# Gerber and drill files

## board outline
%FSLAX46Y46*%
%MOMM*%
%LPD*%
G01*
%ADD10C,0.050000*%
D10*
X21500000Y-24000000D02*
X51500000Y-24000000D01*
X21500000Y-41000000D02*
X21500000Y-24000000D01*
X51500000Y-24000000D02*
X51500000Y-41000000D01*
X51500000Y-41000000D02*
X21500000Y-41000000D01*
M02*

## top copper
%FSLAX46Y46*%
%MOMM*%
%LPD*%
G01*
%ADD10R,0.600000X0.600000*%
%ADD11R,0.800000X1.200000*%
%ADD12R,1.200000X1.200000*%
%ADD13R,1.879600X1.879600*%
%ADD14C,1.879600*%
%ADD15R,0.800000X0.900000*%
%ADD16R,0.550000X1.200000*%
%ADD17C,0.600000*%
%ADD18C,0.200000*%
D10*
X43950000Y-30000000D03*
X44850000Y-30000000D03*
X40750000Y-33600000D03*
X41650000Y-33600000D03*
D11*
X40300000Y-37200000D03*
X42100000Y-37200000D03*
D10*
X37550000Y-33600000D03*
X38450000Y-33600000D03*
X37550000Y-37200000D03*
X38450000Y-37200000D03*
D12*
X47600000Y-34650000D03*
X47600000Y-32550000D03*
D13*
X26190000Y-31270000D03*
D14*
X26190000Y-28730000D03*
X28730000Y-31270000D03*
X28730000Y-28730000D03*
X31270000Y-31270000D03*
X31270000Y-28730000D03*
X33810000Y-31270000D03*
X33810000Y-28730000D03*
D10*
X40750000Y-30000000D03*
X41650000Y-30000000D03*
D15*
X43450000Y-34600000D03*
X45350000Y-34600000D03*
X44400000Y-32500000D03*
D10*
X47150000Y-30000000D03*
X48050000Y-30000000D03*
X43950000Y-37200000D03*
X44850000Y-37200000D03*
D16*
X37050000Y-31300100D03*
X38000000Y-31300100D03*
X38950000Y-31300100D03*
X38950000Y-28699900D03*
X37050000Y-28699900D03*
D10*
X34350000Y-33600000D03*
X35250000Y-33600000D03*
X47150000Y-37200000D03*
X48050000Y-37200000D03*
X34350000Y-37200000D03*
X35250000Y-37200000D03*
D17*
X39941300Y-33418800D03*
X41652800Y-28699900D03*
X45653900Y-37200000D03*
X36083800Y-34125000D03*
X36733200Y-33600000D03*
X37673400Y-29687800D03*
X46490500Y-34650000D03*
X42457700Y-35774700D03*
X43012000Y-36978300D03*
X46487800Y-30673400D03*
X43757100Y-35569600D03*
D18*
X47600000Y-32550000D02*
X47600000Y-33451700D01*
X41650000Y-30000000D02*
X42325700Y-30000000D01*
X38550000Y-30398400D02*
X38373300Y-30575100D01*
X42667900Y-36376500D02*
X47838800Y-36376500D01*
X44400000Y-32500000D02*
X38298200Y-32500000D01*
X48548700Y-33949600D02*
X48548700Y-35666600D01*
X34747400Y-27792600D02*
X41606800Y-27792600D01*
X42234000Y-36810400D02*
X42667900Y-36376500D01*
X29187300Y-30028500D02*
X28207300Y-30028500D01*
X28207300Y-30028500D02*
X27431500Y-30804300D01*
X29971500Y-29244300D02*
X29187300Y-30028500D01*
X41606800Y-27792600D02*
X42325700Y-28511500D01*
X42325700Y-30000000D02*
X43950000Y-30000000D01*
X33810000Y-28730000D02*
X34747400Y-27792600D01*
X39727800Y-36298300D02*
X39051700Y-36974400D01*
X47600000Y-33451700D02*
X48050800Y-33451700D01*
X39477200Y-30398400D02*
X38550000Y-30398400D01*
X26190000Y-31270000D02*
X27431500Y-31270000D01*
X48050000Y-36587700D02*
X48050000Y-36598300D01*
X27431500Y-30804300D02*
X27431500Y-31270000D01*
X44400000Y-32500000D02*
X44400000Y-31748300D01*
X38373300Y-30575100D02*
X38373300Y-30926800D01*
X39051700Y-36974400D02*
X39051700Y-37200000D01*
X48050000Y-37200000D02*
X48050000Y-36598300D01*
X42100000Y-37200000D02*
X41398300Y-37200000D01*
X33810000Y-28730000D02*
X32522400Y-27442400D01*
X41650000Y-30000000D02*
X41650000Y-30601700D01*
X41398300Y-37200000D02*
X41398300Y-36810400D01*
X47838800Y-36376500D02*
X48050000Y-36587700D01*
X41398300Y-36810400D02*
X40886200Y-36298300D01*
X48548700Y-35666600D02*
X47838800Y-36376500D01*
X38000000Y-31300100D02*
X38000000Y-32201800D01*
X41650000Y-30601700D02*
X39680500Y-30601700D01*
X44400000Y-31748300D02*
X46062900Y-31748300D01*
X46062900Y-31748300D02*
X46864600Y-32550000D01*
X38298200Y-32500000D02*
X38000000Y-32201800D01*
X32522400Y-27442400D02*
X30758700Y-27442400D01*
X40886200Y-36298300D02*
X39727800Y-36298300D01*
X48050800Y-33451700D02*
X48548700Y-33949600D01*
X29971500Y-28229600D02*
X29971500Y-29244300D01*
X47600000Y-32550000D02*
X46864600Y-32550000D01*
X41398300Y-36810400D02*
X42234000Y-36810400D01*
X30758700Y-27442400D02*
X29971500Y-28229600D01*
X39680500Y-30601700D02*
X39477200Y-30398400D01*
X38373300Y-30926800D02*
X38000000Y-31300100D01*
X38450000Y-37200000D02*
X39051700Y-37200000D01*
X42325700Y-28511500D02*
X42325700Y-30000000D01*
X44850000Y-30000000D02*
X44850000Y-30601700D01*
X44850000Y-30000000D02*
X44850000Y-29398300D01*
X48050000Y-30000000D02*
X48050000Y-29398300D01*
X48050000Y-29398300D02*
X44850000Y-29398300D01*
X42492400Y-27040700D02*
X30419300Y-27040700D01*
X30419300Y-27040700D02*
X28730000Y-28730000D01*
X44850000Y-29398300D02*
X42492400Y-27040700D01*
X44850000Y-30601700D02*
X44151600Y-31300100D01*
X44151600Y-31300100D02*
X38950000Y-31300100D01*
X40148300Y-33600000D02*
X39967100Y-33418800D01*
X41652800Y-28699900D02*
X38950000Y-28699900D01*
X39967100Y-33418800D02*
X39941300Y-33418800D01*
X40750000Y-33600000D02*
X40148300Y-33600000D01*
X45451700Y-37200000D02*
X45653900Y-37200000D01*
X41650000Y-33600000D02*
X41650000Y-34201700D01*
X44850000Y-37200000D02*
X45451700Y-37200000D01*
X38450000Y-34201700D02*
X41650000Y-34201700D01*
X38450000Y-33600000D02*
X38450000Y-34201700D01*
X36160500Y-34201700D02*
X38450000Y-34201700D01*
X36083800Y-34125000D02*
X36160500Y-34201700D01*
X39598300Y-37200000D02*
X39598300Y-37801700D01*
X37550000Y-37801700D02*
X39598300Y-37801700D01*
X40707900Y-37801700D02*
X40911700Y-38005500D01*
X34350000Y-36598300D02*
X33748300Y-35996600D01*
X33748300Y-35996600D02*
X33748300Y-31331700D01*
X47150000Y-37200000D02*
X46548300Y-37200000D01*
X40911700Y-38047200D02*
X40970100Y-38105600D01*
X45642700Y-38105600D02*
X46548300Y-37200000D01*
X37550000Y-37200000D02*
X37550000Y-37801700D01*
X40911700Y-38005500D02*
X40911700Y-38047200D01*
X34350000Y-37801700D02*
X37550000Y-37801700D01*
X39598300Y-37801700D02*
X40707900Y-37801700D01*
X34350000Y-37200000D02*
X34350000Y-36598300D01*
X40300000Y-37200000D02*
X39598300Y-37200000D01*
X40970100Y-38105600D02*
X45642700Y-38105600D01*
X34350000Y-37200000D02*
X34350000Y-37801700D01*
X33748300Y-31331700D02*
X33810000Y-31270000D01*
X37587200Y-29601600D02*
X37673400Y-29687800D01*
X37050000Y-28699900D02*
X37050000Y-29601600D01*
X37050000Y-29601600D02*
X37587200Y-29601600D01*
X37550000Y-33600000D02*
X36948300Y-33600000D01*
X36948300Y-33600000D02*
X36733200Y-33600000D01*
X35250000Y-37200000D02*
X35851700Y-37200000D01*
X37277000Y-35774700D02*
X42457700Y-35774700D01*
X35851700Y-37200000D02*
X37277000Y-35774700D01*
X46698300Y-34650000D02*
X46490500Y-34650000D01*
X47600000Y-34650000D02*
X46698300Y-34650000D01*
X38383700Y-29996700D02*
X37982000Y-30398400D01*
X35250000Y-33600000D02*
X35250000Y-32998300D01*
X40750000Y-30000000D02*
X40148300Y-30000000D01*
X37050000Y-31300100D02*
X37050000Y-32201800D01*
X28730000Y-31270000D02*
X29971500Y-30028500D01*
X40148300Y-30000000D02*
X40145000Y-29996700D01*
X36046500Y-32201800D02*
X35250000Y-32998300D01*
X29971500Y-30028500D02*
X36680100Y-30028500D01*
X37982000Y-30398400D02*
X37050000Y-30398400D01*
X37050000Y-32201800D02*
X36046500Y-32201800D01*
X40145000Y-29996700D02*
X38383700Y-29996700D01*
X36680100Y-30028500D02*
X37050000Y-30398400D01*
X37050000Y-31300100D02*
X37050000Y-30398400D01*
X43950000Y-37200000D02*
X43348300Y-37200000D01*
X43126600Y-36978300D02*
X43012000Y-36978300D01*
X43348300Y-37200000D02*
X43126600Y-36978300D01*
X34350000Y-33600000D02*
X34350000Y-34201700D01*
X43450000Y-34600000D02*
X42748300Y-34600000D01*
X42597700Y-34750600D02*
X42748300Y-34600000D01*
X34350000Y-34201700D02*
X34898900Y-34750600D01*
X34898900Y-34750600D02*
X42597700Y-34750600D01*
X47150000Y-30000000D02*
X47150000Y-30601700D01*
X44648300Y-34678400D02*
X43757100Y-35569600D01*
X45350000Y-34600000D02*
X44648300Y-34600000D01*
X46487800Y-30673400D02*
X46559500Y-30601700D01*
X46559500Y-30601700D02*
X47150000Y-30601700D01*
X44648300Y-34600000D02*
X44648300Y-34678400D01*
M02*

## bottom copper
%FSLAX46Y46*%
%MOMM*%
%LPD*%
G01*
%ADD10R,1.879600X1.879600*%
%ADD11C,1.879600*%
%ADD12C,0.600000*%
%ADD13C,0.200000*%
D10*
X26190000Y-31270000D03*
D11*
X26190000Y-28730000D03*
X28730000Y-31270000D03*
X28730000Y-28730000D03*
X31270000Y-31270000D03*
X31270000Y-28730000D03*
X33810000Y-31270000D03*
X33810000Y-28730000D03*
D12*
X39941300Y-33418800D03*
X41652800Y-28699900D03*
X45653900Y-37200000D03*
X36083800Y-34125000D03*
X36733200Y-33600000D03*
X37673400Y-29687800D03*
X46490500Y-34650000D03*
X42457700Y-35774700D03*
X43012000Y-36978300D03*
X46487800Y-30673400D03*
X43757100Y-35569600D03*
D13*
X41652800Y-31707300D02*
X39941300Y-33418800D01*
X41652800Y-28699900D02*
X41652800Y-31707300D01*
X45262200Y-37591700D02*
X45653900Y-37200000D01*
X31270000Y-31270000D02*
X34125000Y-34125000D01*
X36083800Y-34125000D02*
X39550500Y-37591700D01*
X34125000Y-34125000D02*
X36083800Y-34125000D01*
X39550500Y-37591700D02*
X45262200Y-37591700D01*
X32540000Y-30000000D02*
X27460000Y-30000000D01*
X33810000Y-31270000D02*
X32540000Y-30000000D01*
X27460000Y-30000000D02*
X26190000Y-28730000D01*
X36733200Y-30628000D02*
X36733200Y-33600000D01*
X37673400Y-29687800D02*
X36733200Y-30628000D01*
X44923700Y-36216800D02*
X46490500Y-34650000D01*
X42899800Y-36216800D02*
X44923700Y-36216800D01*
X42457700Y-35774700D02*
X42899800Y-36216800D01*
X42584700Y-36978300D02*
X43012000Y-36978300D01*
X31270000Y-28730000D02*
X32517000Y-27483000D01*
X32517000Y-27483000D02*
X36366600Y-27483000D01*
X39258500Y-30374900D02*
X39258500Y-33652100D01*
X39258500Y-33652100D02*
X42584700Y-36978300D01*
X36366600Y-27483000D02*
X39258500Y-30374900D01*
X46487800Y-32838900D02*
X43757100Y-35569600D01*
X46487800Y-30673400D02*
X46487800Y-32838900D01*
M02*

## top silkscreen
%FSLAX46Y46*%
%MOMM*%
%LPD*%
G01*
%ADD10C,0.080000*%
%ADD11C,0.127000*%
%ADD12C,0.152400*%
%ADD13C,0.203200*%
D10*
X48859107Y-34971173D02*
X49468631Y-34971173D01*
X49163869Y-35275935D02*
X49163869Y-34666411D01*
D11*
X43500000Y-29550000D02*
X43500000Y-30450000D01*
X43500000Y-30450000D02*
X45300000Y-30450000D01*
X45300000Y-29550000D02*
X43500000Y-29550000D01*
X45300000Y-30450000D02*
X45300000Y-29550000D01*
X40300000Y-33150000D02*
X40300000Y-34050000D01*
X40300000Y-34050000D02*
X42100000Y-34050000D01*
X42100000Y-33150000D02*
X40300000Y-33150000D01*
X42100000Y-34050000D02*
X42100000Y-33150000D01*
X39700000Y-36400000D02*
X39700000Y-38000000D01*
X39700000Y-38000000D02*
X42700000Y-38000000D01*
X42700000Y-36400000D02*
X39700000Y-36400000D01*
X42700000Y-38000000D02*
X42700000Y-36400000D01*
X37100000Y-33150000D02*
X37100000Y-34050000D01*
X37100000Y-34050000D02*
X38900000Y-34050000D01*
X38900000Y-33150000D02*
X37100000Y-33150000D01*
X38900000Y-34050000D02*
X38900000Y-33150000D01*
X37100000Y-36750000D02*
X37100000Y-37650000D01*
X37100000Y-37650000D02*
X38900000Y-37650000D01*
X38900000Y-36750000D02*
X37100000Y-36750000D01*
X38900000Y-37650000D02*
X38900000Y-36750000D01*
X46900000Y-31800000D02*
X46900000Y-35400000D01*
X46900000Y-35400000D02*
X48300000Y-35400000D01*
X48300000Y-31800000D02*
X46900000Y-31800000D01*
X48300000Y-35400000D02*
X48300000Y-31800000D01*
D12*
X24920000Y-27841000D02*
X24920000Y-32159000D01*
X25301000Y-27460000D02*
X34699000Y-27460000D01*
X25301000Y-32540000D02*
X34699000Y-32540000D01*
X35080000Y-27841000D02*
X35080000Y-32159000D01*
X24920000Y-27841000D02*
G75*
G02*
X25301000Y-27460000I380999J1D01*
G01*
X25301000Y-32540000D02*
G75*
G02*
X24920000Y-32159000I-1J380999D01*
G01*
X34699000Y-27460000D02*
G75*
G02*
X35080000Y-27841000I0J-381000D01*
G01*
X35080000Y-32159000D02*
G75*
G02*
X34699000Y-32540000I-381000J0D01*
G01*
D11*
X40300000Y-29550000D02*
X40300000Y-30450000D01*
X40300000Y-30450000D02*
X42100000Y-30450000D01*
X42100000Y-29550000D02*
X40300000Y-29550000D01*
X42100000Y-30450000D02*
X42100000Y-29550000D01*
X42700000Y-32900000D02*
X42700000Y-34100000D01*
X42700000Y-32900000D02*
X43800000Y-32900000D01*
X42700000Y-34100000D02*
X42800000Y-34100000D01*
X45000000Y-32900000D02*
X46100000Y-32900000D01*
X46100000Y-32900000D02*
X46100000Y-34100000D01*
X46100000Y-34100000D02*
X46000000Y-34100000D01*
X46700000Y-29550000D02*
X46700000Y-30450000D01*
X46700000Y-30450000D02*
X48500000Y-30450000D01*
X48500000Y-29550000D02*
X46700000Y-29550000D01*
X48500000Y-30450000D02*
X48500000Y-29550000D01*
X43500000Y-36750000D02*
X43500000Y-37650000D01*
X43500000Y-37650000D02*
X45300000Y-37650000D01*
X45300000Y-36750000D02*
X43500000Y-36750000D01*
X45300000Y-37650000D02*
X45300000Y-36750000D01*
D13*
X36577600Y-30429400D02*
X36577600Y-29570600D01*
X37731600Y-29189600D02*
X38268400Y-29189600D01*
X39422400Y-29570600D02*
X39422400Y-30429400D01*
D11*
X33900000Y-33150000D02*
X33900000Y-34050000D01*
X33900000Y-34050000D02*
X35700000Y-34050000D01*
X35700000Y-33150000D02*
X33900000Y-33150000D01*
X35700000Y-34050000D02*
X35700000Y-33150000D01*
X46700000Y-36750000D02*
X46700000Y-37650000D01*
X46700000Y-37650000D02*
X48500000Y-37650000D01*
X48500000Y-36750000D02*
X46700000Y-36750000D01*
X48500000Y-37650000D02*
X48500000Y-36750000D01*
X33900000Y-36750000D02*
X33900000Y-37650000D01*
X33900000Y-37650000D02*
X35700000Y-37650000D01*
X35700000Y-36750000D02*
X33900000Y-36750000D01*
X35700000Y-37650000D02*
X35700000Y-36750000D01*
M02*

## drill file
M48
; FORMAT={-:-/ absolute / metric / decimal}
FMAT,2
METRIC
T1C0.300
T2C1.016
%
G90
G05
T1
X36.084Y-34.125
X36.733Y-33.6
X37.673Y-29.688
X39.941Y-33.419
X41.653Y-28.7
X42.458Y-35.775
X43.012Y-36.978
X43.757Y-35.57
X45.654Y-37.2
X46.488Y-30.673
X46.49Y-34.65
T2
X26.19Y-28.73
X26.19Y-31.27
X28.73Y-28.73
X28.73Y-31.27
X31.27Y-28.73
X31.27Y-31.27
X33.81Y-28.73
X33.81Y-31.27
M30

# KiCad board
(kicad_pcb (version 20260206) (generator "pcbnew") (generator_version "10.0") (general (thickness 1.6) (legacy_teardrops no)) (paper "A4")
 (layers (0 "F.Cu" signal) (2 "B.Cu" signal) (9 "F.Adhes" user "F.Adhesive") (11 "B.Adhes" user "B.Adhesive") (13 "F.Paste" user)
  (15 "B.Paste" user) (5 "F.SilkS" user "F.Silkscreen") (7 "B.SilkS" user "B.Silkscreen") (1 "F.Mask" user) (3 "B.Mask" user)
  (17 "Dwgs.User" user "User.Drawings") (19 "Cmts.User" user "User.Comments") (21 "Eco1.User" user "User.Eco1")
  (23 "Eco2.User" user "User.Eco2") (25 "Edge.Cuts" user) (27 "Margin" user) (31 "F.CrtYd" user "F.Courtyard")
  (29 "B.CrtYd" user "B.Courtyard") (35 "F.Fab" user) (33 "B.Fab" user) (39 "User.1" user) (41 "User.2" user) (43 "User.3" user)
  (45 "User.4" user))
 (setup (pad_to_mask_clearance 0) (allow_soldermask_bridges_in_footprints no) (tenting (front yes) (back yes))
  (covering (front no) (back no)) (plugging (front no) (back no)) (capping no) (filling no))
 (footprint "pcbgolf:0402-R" (layer "F.Cu") (at 44.4 30)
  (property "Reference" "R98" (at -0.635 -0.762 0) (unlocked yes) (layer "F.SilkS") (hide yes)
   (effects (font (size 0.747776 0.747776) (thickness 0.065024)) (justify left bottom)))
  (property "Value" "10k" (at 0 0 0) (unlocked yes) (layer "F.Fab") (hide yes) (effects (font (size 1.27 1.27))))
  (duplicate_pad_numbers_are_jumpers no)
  (fp_line (start -0.9 -0.45) (end -0.9 0.45) (stroke (width 0.127) (type solid)) (layer "F.SilkS"))
  (fp_line (start -0.9 0.45) (end 0.9 0.45) (stroke (width 0.127) (type solid)) (layer "F.SilkS"))
  (fp_line (start 0.9 -0.45) (end -0.9 -0.45) (stroke (width 0.127) (type solid)) (layer "F.SilkS"))
  (fp_line (start 0.9 0.45) (end 0.9 -0.45) (stroke (width 0.127) (type solid)) (layer "F.SilkS"))
  (pad "1" smd rect (at -0.45 0) (size 0.6 0.6) (layers "F.Cu" "F.Mask" "F.Paste") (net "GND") (solder_mask_margin 0.0508)
   (solder_paste_margin 0) (thermal_bridge_angle 0))
  (pad "2" smd rect (at 0.45 0) (size 0.6 0.6) (layers "F.Cu" "F.Mask" "F.Paste") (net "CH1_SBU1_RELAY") (solder_mask_margin 0.0508)
   (solder_paste_margin 0) (thermal_bridge_angle 0)))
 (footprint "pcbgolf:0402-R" (layer "F.Cu") (at 41.2 33.6)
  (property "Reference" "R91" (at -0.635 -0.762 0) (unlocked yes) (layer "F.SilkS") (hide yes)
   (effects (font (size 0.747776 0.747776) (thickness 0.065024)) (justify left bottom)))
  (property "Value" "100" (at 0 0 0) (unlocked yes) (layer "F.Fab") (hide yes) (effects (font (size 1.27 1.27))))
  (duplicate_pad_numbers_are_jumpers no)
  (fp_line (start -0.9 -0.45) (end -0.9 0.45) (stroke (width 0.127) (type solid)) (layer "F.SilkS"))
  (fp_line (start -0.9 0.45) (end 0.9 0.45) (stroke (width 0.127) (type solid)) (layer "F.SilkS"))
  (fp_line (start 0.9 -0.45) (end -0.9 -0.45) (stroke (width 0.127) (type solid)) (layer "F.SilkS"))
  (fp_line (start 0.9 0.45) (end 0.9 -0.45) (stroke (width 0.127) (type solid)) (layer "F.SilkS"))
  (pad "1" smd rect (at -0.45 0) (size 0.6 0.6) (layers "F.Cu" "F.Mask" "F.Paste") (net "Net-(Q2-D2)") (solder_mask_margin 0.0508)
   (solder_paste_margin 0) (thermal_bridge_angle 0))
  (pad "2" smd rect (at 0.45 0) (size 0.6 0.6) (layers "F.Cu" "F.Mask" "F.Paste") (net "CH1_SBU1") (solder_mask_margin 0.0508)
   (solder_paste_margin 0) (thermal_bridge_angle 0)))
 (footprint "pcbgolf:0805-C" (layer "F.Cu") (at 41.2 37.2)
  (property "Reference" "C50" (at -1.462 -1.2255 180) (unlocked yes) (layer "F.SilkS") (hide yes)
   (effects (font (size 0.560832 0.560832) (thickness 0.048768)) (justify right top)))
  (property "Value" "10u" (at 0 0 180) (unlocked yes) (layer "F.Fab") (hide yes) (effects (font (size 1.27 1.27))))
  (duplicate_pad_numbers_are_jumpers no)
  (fp_line (start -1.5 -0.8) (end -1.5 0.8) (stroke (width 0.127) (type solid)) (layer "F.SilkS"))
  (fp_line (start -1.5 0.8) (end 1.5 0.8) (stroke (width 0.127) (type solid)) (layer "F.SilkS"))
  (fp_line (start 1.5 -0.8) (end -1.5 -0.8) (stroke (width 0.127) (type solid)) (layer "F.SilkS"))
  (fp_line (start 1.5 0.8) (end 1.5 -0.8) (stroke (width 0.127) (type solid)) (layer "F.SilkS"))
  (pad "1" smd rect (at -0.9 0) (size 0.8 1.2) (layers "F.Cu" "F.Mask" "F.Paste") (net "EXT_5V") (solder_mask_margin 0.0508)
   (solder_paste_margin 0) (thermal_bridge_angle 0))
  (pad "2" smd rect (at 0.9 0) (size 0.8 1.2) (layers "F.Cu" "F.Mask" "F.Paste") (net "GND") (solder_mask_margin 0.0508)
   (solder_paste_margin 0) (thermal_bridge_angle 0)))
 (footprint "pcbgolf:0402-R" (layer "F.Cu") (at 38 33.6)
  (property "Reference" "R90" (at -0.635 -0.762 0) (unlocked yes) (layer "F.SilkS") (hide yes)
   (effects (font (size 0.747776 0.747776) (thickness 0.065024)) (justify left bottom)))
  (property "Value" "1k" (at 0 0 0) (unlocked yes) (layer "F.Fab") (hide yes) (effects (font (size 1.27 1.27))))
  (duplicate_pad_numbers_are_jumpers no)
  (fp_line (start -0.9 -0.45) (end -0.9 0.45) (stroke (width 0.127) (type solid)) (layer "F.SilkS"))
  (fp_line (start -0.9 0.45) (end 0.9 0.45) (stroke (width 0.127) (type solid)) (layer "F.SilkS"))
  (fp_line (start 0.9 -0.45) (end -0.9 -0.45) (stroke (width 0.127) (type solid)) (layer "F.SilkS"))
  (fp_line (start 0.9 0.45) (end 0.9 -0.45) (stroke (width 0.127) (type solid)) (layer "F.SilkS"))
  (pad "1" smd rect (at -0.45 0) (size 0.6 0.6) (layers "F.Cu" "F.Mask" "F.Paste") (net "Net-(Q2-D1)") (solder_mask_margin 0.0508)
   (solder_paste_margin 0) (thermal_bridge_angle 0))
  (pad "2" smd rect (at 0.45 0) (size 0.6 0.6) (layers "F.Cu" "F.Mask" "F.Paste") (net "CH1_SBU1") (solder_mask_margin 0.0508)
   (solder_paste_margin 0) (thermal_bridge_angle 0)))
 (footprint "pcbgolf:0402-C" (layer "F.Cu") (at 38 37.2)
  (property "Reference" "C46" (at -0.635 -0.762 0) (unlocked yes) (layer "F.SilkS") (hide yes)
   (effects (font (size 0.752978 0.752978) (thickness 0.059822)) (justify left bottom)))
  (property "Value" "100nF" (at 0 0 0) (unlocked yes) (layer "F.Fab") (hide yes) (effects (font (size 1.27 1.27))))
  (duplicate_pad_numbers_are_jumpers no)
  (fp_line (start -0.9 -0.45) (end -0.9 0.45) (stroke (width 0.127) (type solid)) (layer "F.SilkS"))
  (fp_line (start -0.9 0.45) (end 0.9 0.45) (stroke (width 0.127) (type solid)) (layer "F.SilkS"))
  (fp_line (start 0.9 -0.45) (end -0.9 -0.45) (stroke (width 0.127) (type solid)) (layer "F.SilkS"))
  (fp_line (start 0.9 0.45) (end 0.9 -0.45) (stroke (width 0.127) (type solid)) (layer "F.SilkS"))
  (pad "1" smd rect (at -0.45 0) (size 0.6 0.6) (layers "F.Cu" "F.Mask" "F.Paste") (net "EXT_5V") (solder_mask_margin 0.0508)
   (solder_paste_margin 0) (thermal_bridge_angle 0))
  (pad "2" smd rect (at 0.45 0) (size 0.6 0.6) (layers "F.Cu" "F.Mask" "F.Paste") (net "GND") (solder_mask_margin 0.0508)
   (solder_paste_margin 0) (thermal_bridge_angle 0)))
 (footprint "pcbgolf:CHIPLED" (layer "F.Cu") (at 47.6 33.6)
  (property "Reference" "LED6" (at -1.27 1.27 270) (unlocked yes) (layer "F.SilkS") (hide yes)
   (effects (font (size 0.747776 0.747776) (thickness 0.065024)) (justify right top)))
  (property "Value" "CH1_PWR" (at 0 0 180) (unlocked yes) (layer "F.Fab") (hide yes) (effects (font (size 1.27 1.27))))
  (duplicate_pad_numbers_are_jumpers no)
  (fp_line (start -0.7 -1.8) (end -0.7 1.8) (stroke (width 0.127) (type solid)) (layer "F.SilkS"))
  (fp_line (start -0.7 1.8) (end 0.7 1.8) (stroke (width 0.127) (type solid)) (layer "F.SilkS"))
  (fp_line (start 0.7 -1.8) (end -0.7 -1.8) (stroke (width 0.127) (type solid)) (layer "F.SilkS"))
  (fp_line (start 0.7 1.8) (end 0.7 -1.8) (stroke (width 0.127) (type solid)) (layer "F.SilkS"))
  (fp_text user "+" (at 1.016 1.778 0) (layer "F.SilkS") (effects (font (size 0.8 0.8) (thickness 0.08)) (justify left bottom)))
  (pad "A" smd rect (at 0 1.05) (size 1.2 1.2) (layers "F.Cu" "F.Mask" "F.Paste") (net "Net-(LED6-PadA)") (solder_mask_margin 0.0508)
   (solder_paste_margin 0) (thermal_bridge_angle 0))
  (pad "C" smd rect (at 0 -1.05) (size 1.2 1.2) (layers "F.Cu" "F.Mask" "F.Paste") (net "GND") (solder_mask_margin 0.0508)
   (solder_paste_margin 0) (thermal_bridge_angle 0)))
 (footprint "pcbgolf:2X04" (layer "F.Cu") (at 30 30)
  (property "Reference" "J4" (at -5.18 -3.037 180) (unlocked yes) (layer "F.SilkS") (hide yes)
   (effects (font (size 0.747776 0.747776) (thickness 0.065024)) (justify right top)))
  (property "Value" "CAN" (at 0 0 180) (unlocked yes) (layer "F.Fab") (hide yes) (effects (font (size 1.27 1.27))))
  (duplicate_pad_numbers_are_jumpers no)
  (fp_line (start -5.08 -2.159) (end -5.08 2.159) (stroke (width 0.1524) (type solid)) (layer "F.SilkS"))
  (fp_line (start -4.699 -2.54) (end 4.699 -2.54) (stroke (width 0.1524) (type solid)) (layer "F.SilkS"))
  (fp_line (start -4.699 2.54) (end 4.699 2.54) (stroke (width 0.1524) (type solid)) (layer "F.SilkS"))
  (fp_line (start 5.08 -2.159) (end 5.08 2.159) (stroke (width 0.1524) (type solid)) (layer "F.SilkS"))
  (fp_arc (start -5.08 -2.159) (mid -4.968408 -2.428408) (end -4.699 -2.54) (stroke (width 0.1524) (type solid)) (layer "F.SilkS"))
  (fp_arc (start -4.699 2.54) (mid -4.968408 2.428408) (end -5.08 2.159) (stroke (width 0.1524) (type solid)) (layer "F.SilkS"))
  (fp_arc (start 4.699 -2.54) (mid 4.968408 -2.428408) (end 5.08 -2.159) (stroke (width 0.1524) (type solid)) (layer "F.SilkS"))
  (fp_arc (start 5.08 2.159) (mid 4.968408 2.428408) (end 4.699 2.54) (stroke (width 0.1524) (type solid)) (layer "F.SilkS"))
  (pad "1" thru_hole rect (at -3.81 1.27 90) (size 1.8796 1.8796) (drill 1.016) (layers "*.Cu" "*.Mask") (remove_unused_layers no)
   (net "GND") (solder_mask_margin 0.0508) (thermal_bridge_angle 0))
  (pad "2" thru_hole circle (at -3.81 -1.27 90) (size 1.8796 1.8796) (drill 1.016) (layers "*.Cu" "*.Mask") (remove_unused_layers no)
   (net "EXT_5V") (solder_mask_margin 0.0508) (thermal_bridge_angle 0))
  (pad "3" thru_hole circle (at -1.27 1.27 90) (size 1.8796 1.8796) (drill 1.016) (layers "*.Cu" "*.Mask") (remove_unused_layers no)
   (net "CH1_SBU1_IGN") (solder_mask_margin 0.0508) (thermal_bridge_angle 0))
  (pad "4" thru_hole circle (at -1.27 -1.27 90) (size 1.8796 1.8796) (drill 1.016) (layers "*.Cu" "*.Mask") (remove_unused_layers no)
   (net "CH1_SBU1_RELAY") (solder_mask_margin 0.0508) (thermal_bridge_angle 0))
  (pad "5" thru_hole circle (at 1.27 1.27 90) (size 1.8796 1.8796) (drill 1.016) (layers "*.Cu" "*.Mask") (remove_unused_layers no)
   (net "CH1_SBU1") (solder_mask_margin 0.0508) (thermal_bridge_angle 0))
  (pad "6" thru_hole circle (at 1.27 -1.27 90) (size 1.8796 1.8796) (drill 1.016) (layers "*.Cu" "*.Mask") (remove_unused_layers no)
   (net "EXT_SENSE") (solder_mask_margin 0.0508) (thermal_bridge_angle 0))
  (pad "7" thru_hole circle (at 3.81 1.27 90) (size 1.8796 1.8796) (drill 1.016) (layers "*.Cu" "*.Mask") (remove_unused_layers no)
   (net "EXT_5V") (solder_mask_margin 0.0508) (thermal_bridge_angle 0))
  (pad "8" thru_hole circle (at 3.81 -1.27 90) (size 1.8796 1.8796) (drill 1.016) (layers "*.Cu" "*.Mask") (remove_unused_layers no)
   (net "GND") (solder_mask_margin 0.0508) (thermal_bridge_angle 0)))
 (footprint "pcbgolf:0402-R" (layer "F.Cu") (at 41.2 30)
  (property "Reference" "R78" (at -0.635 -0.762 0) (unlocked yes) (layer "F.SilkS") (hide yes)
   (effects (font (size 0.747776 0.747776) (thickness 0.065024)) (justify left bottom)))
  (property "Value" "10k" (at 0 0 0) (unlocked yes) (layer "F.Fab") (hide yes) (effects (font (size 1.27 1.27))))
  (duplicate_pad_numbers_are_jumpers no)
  (fp_line (start -0.9 -0.45) (end -0.9 0.45) (stroke (width 0.127) (type solid)) (layer "F.SilkS"))
  (fp_line (start -0.9 0.45) (end 0.9 0.45) (stroke (width 0.127) (type solid)) (layer "F.SilkS"))
  (fp_line (start 0.9 -0.45) (end -0.9 -0.45) (stroke (width 0.127) (type solid)) (layer "F.SilkS"))
  (fp_line (start 0.9 0.45) (end 0.9 -0.45) (stroke (width 0.127) (type solid)) (layer "F.SilkS"))
  (pad "1" smd rect (at -0.45 0) (size 0.6 0.6) (layers "F.Cu" "F.Mask" "F.Paste") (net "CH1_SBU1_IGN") (solder_mask_margin 0.0508)
   (solder_paste_margin 0) (thermal_bridge_angle 0))
  (pad "2" smd rect (at 0.45 0) (size 0.6 0.6) (layers "F.Cu" "F.Mask" "F.Paste") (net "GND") (solder_mask_margin 0.0508)
   (solder_paste_margin 0) (thermal_bridge_angle 0)))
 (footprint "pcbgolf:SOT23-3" (layer "F.Cu") (at 44.4 33.6)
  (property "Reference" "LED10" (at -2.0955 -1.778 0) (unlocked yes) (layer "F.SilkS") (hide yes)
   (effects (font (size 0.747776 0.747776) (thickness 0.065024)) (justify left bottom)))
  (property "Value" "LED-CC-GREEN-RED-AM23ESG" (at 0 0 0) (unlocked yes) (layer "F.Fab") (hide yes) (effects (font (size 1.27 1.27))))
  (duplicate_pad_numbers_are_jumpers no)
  (fp_line (start -1.7 -0.7) (end -1.7 0.5) (stroke (width 0.127) (type solid)) (layer "F.SilkS"))
  (fp_line (start -1.7 -0.7) (end -0.6 -0.7) (stroke (width 0.127) (type solid)) (layer "F.SilkS"))
  (fp_line (start -1.7 0.5) (end -1.6 0.5) (stroke (width 0.127) (type solid)) (layer "F.SilkS"))
  (fp_line (start 0.6 -0.7) (end 1.7 -0.7) (stroke (width 0.127) (type solid)) (layer "F.SilkS"))
  (fp_line (start 1.7 -0.7) (end 1.7 0.5) (stroke (width 0.127) (type solid)) (layer "F.SilkS"))
  (fp_line (start 1.7 0.5) (end 1.6 0.5) (stroke (width 0.127) (type solid)) (layer "F.SilkS"))
  (pad "1" smd rect (at -0.95 1) (size 0.8 0.9) (layers "F.Cu" "F.Mask" "F.Paste") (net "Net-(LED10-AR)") (solder_mask_margin 0.0508)
   (solder_paste_margin 0) (thermal_bridge_angle 0))
  (pad "2" smd rect (at 0.95 1) (size 0.8 0.9) (layers "F.Cu" "F.Mask" "F.Paste") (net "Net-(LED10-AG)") (solder_mask_margin 0.0508)
   (solder_paste_margin 0) (thermal_bridge_angle 0))
  (pad "3" smd rect (at 0 -1.1) (size 0.8 0.9) (layers "F.Cu" "F.Mask" "F.Paste") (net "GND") (solder_mask_margin 0.0508)
   (solder_paste_margin 0) (thermal_bridge_angle 0)))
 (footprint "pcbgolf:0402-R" (layer "F.Cu") (at 47.6 30)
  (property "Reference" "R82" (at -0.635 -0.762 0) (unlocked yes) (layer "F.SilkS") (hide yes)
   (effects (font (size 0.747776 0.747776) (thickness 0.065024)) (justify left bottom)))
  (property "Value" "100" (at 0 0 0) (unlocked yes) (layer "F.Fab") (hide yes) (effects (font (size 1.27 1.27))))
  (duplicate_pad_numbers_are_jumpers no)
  (fp_line (start -0.9 -0.45) (end -0.9 0.45) (stroke (width 0.127) (type solid)) (layer "F.SilkS"))
  (fp_line (start -0.9 0.45) (end 0.9 0.45) (stroke (width 0.127) (type solid)) (layer "F.SilkS"))
  (fp_line (start 0.9 -0.45) (end -0.9 -0.45) (stroke (width 0.127) (type solid)) (layer "F.SilkS"))
  (fp_line (start 0.9 0.45) (end 0.9 -0.45) (stroke (width 0.127) (type solid)) (layer "F.SilkS"))
  (pad "1" smd rect (at -0.45 0) (size 0.6 0.6) (layers "F.Cu" "F.Mask" "F.Paste") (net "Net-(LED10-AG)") (solder_mask_margin 0.0508)
   (solder_paste_margin 0) (thermal_bridge_angle 0))
  (pad "2" smd rect (at 0.45 0) (size 0.6 0.6) (layers "F.Cu" "F.Mask" "F.Paste") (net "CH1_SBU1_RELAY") (solder_mask_margin 0.0508)
   (solder_paste_margin 0) (thermal_bridge_angle 0)))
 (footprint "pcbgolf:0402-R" (layer "F.Cu") (at 44.4 37.2)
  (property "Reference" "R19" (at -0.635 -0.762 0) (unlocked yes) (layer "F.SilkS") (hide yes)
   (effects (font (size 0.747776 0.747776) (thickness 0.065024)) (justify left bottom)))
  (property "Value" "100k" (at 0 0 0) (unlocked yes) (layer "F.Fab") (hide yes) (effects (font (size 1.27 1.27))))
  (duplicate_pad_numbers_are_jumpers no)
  (fp_line (start -0.9 -0.45) (end -0.9 0.45) (stroke (width 0.127) (type solid)) (layer "F.SilkS"))
  (fp_line (start -0.9 0.45) (end 0.9 0.45) (stroke (width 0.127) (type solid)) (layer "F.SilkS"))
  (fp_line (start 0.9 -0.45) (end -0.9 -0.45) (stroke (width 0.127) (type solid)) (layer "F.SilkS"))
  (fp_line (start 0.9 0.45) (end 0.9 -0.45) (stroke (width 0.127) (type solid)) (layer "F.SilkS"))
  (pad "1" smd rect (at -0.45 0) (size 0.6 0.6) (layers "F.Cu" "F.Mask" "F.Paste") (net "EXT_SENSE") (solder_mask_margin 0.0508)
   (solder_paste_margin 0) (thermal_bridge_angle 0))
  (pad "2" smd rect (at 0.45 0) (size 0.6 0.6) (layers "F.Cu" "F.Mask" "F.Paste") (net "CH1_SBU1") (solder_mask_margin 0.0508)
   (solder_paste_margin 0) (thermal_bridge_angle 0)))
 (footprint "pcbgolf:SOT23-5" (layer "F.Cu") (at 38 30)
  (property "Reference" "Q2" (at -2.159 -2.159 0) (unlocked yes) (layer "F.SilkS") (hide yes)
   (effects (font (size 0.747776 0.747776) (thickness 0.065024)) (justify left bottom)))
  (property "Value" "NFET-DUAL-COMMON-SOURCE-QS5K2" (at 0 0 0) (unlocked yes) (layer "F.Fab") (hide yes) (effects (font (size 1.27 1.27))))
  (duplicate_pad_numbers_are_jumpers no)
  (fp_line (start -1.4224 0.4294) (end -1.4224 -0.4294) (stroke (width 0.2032) (type solid)) (layer "F.SilkS"))
  (fp_line (start -0.2684 -0.8104) (end 0.2684 -0.8104) (stroke (width 0.2032) (type solid)) (layer "F.SilkS"))
  (fp_line (start 1.4224 -0.4294) (end 1.4224 0.4294) (stroke (width 0.2032) (type solid)) (layer "F.SilkS"))
  (pad "1" smd rect (at -0.95 1.3001) (size 0.55 1.2) (layers "F.Cu" "F.Mask" "F.Paste") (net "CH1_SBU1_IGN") (solder_mask_margin 0.0508)
   (solder_paste_margin 0) (thermal_bridge_angle 0))
  (pad "2" smd rect (at 0 1.3001) (size 0.55 1.2) (layers "F.Cu" "F.Mask" "F.Paste") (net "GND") (solder_mask_margin 0.0508)
   (solder_paste_margin 0) (thermal_bridge_angle 0))
  (pad "3" smd rect (at 0.95 1.3001) (size 0.55 1.2) (layers "F.Cu" "F.Mask" "F.Paste") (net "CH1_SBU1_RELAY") (solder_mask_margin 0.0508)
   (solder_paste_margin 0) (thermal_bridge_angle 0))
  (pad "4" smd rect (at 0.95 -1.3001) (size 0.55 1.2) (layers "F.Cu" "F.Mask" "F.Paste") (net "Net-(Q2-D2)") (solder_mask_margin 0.0508)
   (solder_paste_margin 0) (thermal_bridge_angle 0))
  (pad "5" smd rect (at -0.95 -1.3001) (size 0.55 1.2) (layers "F.Cu" "F.Mask" "F.Paste") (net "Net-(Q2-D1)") (solder_mask_margin 0.0508)
   (solder_paste_margin 0) (thermal_bridge_angle 0)))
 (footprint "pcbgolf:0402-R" (layer "F.Cu") (at 34.8 33.6)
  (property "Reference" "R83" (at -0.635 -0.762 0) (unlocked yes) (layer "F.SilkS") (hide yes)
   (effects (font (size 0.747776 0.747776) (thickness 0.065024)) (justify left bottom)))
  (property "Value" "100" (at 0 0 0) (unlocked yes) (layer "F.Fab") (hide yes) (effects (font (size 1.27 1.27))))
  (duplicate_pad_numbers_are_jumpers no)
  (fp_line (start -0.9 -0.45) (end -0.9 0.45) (stroke (width 0.127) (type solid)) (layer "F.SilkS"))
  (fp_line (start -0.9 0.45) (end 0.9 0.45) (stroke (width 0.127) (type solid)) (layer "F.SilkS"))
  (fp_line (start 0.9 -0.45) (end -0.9 -0.45) (stroke (width 0.127) (type solid)) (layer "F.SilkS"))
  (fp_line (start 0.9 0.45) (end 0.9 -0.45) (stroke (width 0.127) (type solid)) (layer "F.SilkS"))
  (pad "1" smd rect (at -0.45 0) (size 0.6 0.6) (layers "F.Cu" "F.Mask" "F.Paste") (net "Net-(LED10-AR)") (solder_mask_margin 0.0508)
   (solder_paste_margin 0) (thermal_bridge_angle 0))
  (pad "2" smd rect (at 0.45 0) (size 0.6 0.6) (layers "F.Cu" "F.Mask" "F.Paste") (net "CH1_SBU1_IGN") (solder_mask_margin 0.0508)
   (solder_paste_margin 0) (thermal_bridge_angle 0)))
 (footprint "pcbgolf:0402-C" (layer "F.Cu") (at 47.6 37.2)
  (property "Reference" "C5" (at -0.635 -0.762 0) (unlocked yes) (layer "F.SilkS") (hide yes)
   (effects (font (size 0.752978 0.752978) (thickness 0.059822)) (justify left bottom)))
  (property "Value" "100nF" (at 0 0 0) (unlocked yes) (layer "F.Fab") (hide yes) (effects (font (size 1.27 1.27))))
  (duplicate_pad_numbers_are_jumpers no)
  (fp_line (start -0.9 -0.45) (end -0.9 0.45) (stroke (width 0.127) (type solid)) (layer "F.SilkS"))
  (fp_line (start -0.9 0.45) (end 0.9 0.45) (stroke (width 0.127) (type solid)) (layer "F.SilkS"))
  (fp_line (start 0.9 -0.45) (end -0.9 -0.45) (stroke (width 0.127) (type solid)) (layer "F.SilkS"))
  (fp_line (start 0.9 0.45) (end 0.9 -0.45) (stroke (width 0.127) (type solid)) (layer "F.SilkS"))
  (pad "1" smd rect (at -0.45 0) (size 0.6 0.6) (layers "F.Cu" "F.Mask" "F.Paste") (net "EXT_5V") (solder_mask_margin 0.0508)
   (solder_paste_margin 0) (thermal_bridge_angle 0))
  (pad "2" smd rect (at 0.45 0) (size 0.6 0.6) (layers "F.Cu" "F.Mask" "F.Paste") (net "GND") (solder_mask_margin 0.0508)
   (solder_paste_margin 0) (thermal_bridge_angle 0)))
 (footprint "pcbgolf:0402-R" (layer "F.Cu") (at 34.8 37.2)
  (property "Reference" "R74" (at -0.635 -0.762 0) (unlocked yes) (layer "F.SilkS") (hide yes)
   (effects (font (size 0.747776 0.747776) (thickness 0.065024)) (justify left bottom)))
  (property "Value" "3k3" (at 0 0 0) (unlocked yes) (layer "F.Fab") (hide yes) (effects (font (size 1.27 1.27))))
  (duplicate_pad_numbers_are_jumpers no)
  (fp_line (start -0.9 -0.45) (end -0.9 0.45) (stroke (width 0.127) (type solid)) (layer "F.SilkS"))
  (fp_line (start -0.9 0.45) (end 0.9 0.45) (stroke (width 0.127) (type solid)) (layer "F.SilkS"))
  (fp_line (start 0.9 -0.45) (end -0.9 -0.45) (stroke (width 0.127) (type solid)) (layer "F.SilkS"))
  (fp_line (start 0.9 0.45) (end 0.9 -0.45) (stroke (width 0.127) (type solid)) (layer "F.SilkS"))
  (pad "1" smd rect (at -0.45 0) (size 0.6 0.6) (layers "F.Cu" "F.Mask" "F.Paste") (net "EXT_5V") (solder_mask_margin 0.0508)
   (solder_paste_margin 0) (thermal_bridge_angle 0))
  (pad "2" smd rect (at 0.45 0) (size 0.6 0.6) (layers "F.Cu" "F.Mask" "F.Paste") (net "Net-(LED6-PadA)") (solder_mask_margin 0.0508)
   (solder_paste_margin 0) (thermal_bridge_angle 0)))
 (gr_line (start 21.5 24) (end 51.5 24) (stroke (width 0.05) (type default)) (layer "Edge.Cuts"))
 (gr_line (start 21.5 41) (end 21.5 24) (stroke (width 0.05) (type default)) (layer "Edge.Cuts"))
 (gr_line (start 51.5 24) (end 51.5 41) (stroke (width 0.05) (type default)) (layer "Edge.Cuts"))
 (gr_line (start 51.5 41) (end 21.5 41) (stroke (width 0.05) (type default)) (layer "Edge.Cuts"))
 (segment (start 47.6 32.55) (end 47.6 33.4517) (width 0.2) (layer "F.Cu") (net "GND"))
 (segment (start 41.65 30) (end 42.3257 30) (width 0.2) (layer "F.Cu") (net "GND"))
 (segment (start 38.55 30.3984) (end 38.3733 30.5751) (width 0.2) (layer "F.Cu") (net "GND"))
 (segment (start 42.6679 36.3765) (end 47.8388 36.3765) (width 0.2) (layer "F.Cu") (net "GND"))
 (segment (start 44.4 32.5) (end 38.2982 32.5) (width 0.2) (layer "F.Cu") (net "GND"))
 (segment (start 48.5487 33.9496) (end 48.5487 35.6666) (width 0.2) (layer "F.Cu") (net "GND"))
 (segment (start 34.7474 27.7926) (end 41.6068 27.7926) (width 0.2) (layer "F.Cu") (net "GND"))
 (segment (start 42.234 36.8104) (end 42.6679 36.3765) (width 0.2) (layer "F.Cu") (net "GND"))
 (segment (start 29.1873 30.0285) (end 28.2073 30.0285) (width 0.2) (layer "F.Cu") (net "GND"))
 (segment (start 28.2073 30.0285) (end 27.4315 30.8043) (width 0.2) (layer "F.Cu") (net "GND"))
 (segment (start 29.9715 29.2443) (end 29.1873 30.0285) (width 0.2) (layer "F.Cu") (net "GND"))
 (segment (start 41.6068 27.7926) (end 42.3257 28.5115) (width 0.2) (layer "F.Cu") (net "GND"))
 (segment (start 42.3257 30) (end 43.95 30) (width 0.2) (layer "F.Cu") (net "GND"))
 (segment (start 33.81 28.73) (end 34.7474 27.7926) (width 0.2) (layer "F.Cu") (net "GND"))
 (segment (start 39.7278 36.2983) (end 39.0517 36.9744) (width 0.2) (layer "F.Cu") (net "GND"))
 (segment (start 47.6 33.4517) (end 48.0508 33.4517) (width 0.2) (layer "F.Cu") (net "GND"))
 (segment (start 39.4772 30.3984) (end 38.55 30.3984) (width 0.2) (layer "F.Cu") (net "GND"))
 (segment (start 26.19 31.27) (end 27.4315 31.27) (width 0.2) (layer "F.Cu") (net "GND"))
 (segment (start 48.05 36.5877) (end 48.05 36.5983) (width 0.2) (layer "F.Cu") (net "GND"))
 (segment (start 27.4315 30.8043) (end 27.4315 31.27) (width 0.2) (layer "F.Cu") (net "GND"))
 (segment (start 44.4 32.5) (end 44.4 31.7483) (width 0.2) (layer "F.Cu") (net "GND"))
 (segment (start 38.3733 30.5751) (end 38.3733 30.9268) (width 0.2) (layer "F.Cu") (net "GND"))
 (segment (start 39.0517 36.9744) (end 39.0517 37.2) (width 0.2) (layer "F.Cu") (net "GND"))
 (segment (start 48.05 37.2) (end 48.05 36.5983) (width 0.2) (layer "F.Cu") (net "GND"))
 (segment (start 42.1 37.2) (end 41.3983 37.2) (width 0.2) (layer "F.Cu") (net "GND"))
 (segment (start 33.81 28.73) (end 32.5224 27.4424) (width 0.2) (layer "F.Cu") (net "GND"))
 (segment (start 41.65 30) (end 41.65 30.6017) (width 0.2) (layer "F.Cu") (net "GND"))
 (segment (start 41.3983 37.2) (end 41.3983 36.8104) (width 0.2) (layer "F.Cu") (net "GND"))
 (segment (start 47.8388 36.3765) (end 48.05 36.5877) (width 0.2) (layer "F.Cu") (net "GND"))
 (segment (start 41.3983 36.8104) (end 40.8862 36.2983) (width 0.2) (layer "F.Cu") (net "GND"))
 (segment (start 48.5487 35.6666) (end 47.8388 36.3765) (width 0.2) (layer "F.Cu") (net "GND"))
 (segment (start 38 31.3001) (end 38 32.2018) (width 0.2) (layer "F.Cu") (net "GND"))
 (segment (start 41.65 30.6017) (end 39.6805 30.6017) (width 0.2) (layer "F.Cu") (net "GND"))
 (segment (start 44.4 31.7483) (end 46.0629 31.7483) (width 0.2) (layer "F.Cu") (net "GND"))
 (segment (start 46.0629 31.7483) (end 46.8646 32.55) (width 0.2) (layer "F.Cu") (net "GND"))
 (segment (start 38.2982 32.5) (end 38 32.2018) (width 0.2) (layer "F.Cu") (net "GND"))
 (segment (start 32.5224 27.4424) (end 30.7587 27.4424) (width 0.2) (layer "F.Cu") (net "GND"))
 (segment (start 40.8862 36.2983) (end 39.7278 36.2983) (width 0.2) (layer "F.Cu") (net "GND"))
 (segment (start 48.0508 33.4517) (end 48.5487 33.9496) (width 0.2) (layer "F.Cu") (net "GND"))
 (segment (start 29.9715 28.2296) (end 29.9715 29.2443) (width 0.2) (layer "F.Cu") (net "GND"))
 (segment (start 47.6 32.55) (end 46.8646 32.55) (width 0.2) (layer "F.Cu") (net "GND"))
 (segment (start 41.3983 36.8104) (end 42.234 36.8104) (width 0.2) (layer "F.Cu") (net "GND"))
 (segment (start 30.7587 27.4424) (end 29.9715 28.2296) (width 0.2) (layer "F.Cu") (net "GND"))
 (segment (start 39.6805 30.6017) (end 39.4772 30.3984) (width 0.2) (layer "F.Cu") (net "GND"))
 (segment (start 38.3733 30.9268) (end 38 31.3001) (width 0.2) (layer "F.Cu") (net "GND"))
 (segment (start 38.45 37.2) (end 39.0517 37.2) (width 0.2) (layer "F.Cu") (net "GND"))
 (segment (start 42.3257 28.5115) (end 42.3257 30) (width 0.2) (layer "F.Cu") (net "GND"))
 (segment (start 44.85 30) (end 44.85 30.6017) (width 0.2) (layer "F.Cu") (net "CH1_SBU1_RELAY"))
 (segment (start 44.85 30) (end 44.85 29.3983) (width 0.2) (layer "F.Cu") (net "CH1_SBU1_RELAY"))
 (segment (start 48.05 30) (end 48.05 29.3983) (width 0.2) (layer "F.Cu") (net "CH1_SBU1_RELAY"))
 (segment (start 48.05 29.3983) (end 44.85 29.3983) (width 0.2) (layer "F.Cu") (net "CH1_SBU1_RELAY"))
 (segment (start 42.4924 27.0407) (end 30.4193 27.0407) (width 0.2) (layer "F.Cu") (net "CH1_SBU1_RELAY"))
 (segment (start 30.4193 27.0407) (end 28.73 28.73) (width 0.2) (layer "F.Cu") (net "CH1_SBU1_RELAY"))
 (segment (start 44.85 29.3983) (end 42.4924 27.0407) (width 0.2) (layer "F.Cu") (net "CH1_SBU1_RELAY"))
 (segment (start 44.85 30.6017) (end 44.1516 31.3001) (width 0.2) (layer "F.Cu") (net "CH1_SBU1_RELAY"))
 (segment (start 44.1516 31.3001) (end 38.95 31.3001) (width 0.2) (layer "F.Cu") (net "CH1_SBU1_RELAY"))
 (segment (start 40.1483 33.6) (end 39.9671 33.4188) (width 0.2) (layer "F.Cu") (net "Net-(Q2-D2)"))
 (segment (start 41.6528 28.6999) (end 38.95 28.6999) (width 0.2) (layer "F.Cu") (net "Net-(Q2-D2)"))
 (segment (start 39.9671 33.4188) (end 39.9413 33.4188) (width 0.2) (layer "F.Cu") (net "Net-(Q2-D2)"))
 (segment (start 40.75 33.6) (end 40.1483 33.6) (width 0.2) (layer "F.Cu") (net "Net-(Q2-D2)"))
 (via (at 39.9413 33.4188) (size 0.6) (drill 0.3) (layers "F.Cu" "B.Cu") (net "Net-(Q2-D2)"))
 (via (at 41.6528 28.6999) (size 0.6) (drill 0.3) (layers "F.Cu" "B.Cu") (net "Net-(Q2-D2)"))
 (segment (start 41.6528 31.7073) (end 39.9413 33.4188) (width 0.2) (layer "B.Cu") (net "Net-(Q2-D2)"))
 (segment (start 41.6528 28.6999) (end 41.6528 31.7073) (width 0.2) (layer "B.Cu") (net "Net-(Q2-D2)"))
 (segment (start 45.4517 37.2) (end 45.6539 37.2) (width 0.2) (layer "F.Cu") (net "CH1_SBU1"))
 (segment (start 41.65 33.6) (end 41.65 34.2017) (width 0.2) (layer "F.Cu") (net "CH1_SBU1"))
 (segment (start 44.85 37.2) (end 45.4517 37.2) (width 0.2) (layer "F.Cu") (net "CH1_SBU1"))
 (segment (start 38.45 34.2017) (end 41.65 34.2017) (width 0.2) (layer "F.Cu") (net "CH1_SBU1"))
 (segment (start 38.45 33.6) (end 38.45 34.2017) (width 0.2) (layer "F.Cu") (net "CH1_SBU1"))
 (segment (start 36.1605 34.2017) (end 38.45 34.2017) (width 0.2) (layer "F.Cu") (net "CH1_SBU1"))
 (segment (start 36.0838 34.125) (end 36.1605 34.2017) (width 0.2) (layer "F.Cu") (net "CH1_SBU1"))
 (via (at 45.6539 37.2) (size 0.6) (drill 0.3) (layers "F.Cu" "B.Cu") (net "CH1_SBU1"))
 (via (at 36.0838 34.125) (size 0.6) (drill 0.3) (layers "F.Cu" "B.Cu") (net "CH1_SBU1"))
 (segment (start 45.2622 37.5917) (end 45.6539 37.2) (width 0.2) (layer "B.Cu") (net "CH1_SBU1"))
 (segment (start 31.27 31.27) (end 34.125 34.125) (width 0.2) (layer "B.Cu") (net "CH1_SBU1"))
 (segment (start 36.0838 34.125) (end 39.5505 37.5917) (width 0.2) (layer "B.Cu") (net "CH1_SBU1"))
 (segment (start 34.125 34.125) (end 36.0838 34.125) (width 0.2) (layer "B.Cu") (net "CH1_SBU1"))
 (segment (start 39.5505 37.5917) (end 45.2622 37.5917) (width 0.2) (layer "B.Cu") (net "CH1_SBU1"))
 (segment (start 39.5983 37.2) (end 39.5983 37.8017) (width 0.2) (layer "F.Cu") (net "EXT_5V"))
 (segment (start 37.55 37.8017) (end 39.5983 37.8017) (width 0.2) (layer "F.Cu") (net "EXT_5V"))
 (segment (start 40.7079 37.8017) (end 40.9117 38.0055) (width 0.2) (layer "F.Cu") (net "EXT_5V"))
 (segment (start 34.35 36.5983) (end 33.7483 35.9966) (width 0.2) (layer "F.Cu") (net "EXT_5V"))
 (segment (start 33.7483 35.9966) (end 33.7483 31.3317) (width 0.2) (layer "F.Cu") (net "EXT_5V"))
 (segment (start 47.15 37.2) (end 46.5483 37.2) (width 0.2) (layer "F.Cu") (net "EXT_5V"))
 (segment (start 40.9117 38.0472) (end 40.9701 38.1056) (width 0.2) (layer "F.Cu") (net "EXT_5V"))
 (segment (start 45.6427 38.1056) (end 46.5483 37.2) (width 0.2) (layer "F.Cu") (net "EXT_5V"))
 (segment (start 37.55 37.2) (end 37.55 37.8017) (width 0.2) (layer "F.Cu") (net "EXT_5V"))
 (segment (start 40.9117 38.0055) (end 40.9117 38.0472) (width 0.2) (layer "F.Cu") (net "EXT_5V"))
 (segment (start 34.35 37.8017) (end 37.55 37.8017) (width 0.2) (layer "F.Cu") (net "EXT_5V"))
 (segment (start 39.5983 37.8017) (end 40.7079 37.8017) (width 0.2) (layer "F.Cu") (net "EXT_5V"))
 (segment (start 34.35 37.2) (end 34.35 36.5983) (width 0.2) (layer "F.Cu") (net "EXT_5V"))
 (segment (start 40.3 37.2) (end 39.5983 37.2) (width 0.2) (layer "F.Cu") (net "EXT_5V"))
 (segment (start 40.9701 38.1056) (end 45.6427 38.1056) (width 0.2) (layer "F.Cu") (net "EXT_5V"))
 (segment (start 34.35 37.2) (end 34.35 37.8017) (width 0.2) (layer "F.Cu") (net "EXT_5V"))
 (segment (start 33.7483 31.3317) (end 33.81 31.27) (width 0.2) (layer "F.Cu") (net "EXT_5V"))
 (segment (start 32.54 30) (end 27.46 30) (width 0.2) (layer "B.Cu") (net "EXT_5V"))
 (segment (start 33.81 31.27) (end 32.54 30) (width 0.2) (layer "B.Cu") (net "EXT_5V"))
 (segment (start 27.46 30) (end 26.19 28.73) (width 0.2) (layer "B.Cu") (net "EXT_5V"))
 (segment (start 37.5872 29.6016) (end 37.6734 29.6878) (width 0.2) (layer "F.Cu") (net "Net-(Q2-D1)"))
 (segment (start 37.05 28.6999) (end 37.05 29.6016) (width 0.2) (layer "F.Cu") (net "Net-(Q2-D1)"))
 (segment (start 37.05 29.6016) (end 37.5872 29.6016) (width 0.2) (layer "F.Cu") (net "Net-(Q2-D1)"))
 (segment (start 37.55 33.6) (end 36.9483 33.6) (width 0.2) (layer "F.Cu") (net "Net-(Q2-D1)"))
 (segment (start 36.9483 33.6) (end 36.7332 33.6) (width 0.2) (layer "F.Cu") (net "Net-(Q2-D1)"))
 (via (at 36.7332 33.6) (size 0.6) (drill 0.3) (layers "F.Cu" "B.Cu") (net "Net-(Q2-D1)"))
 (via (at 37.6734 29.6878) (size 0.6) (drill 0.3) (layers "F.Cu" "B.Cu") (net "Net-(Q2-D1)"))
 (segment (start 36.7332 30.628) (end 36.7332 33.6) (width 0.2) (layer "B.Cu") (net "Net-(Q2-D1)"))
 (segment (start 37.6734 29.6878) (end 36.7332 30.628) (width 0.2) (layer "B.Cu") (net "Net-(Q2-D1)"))
 (segment (start 35.25 37.2) (end 35.8517 37.2) (width 0.2) (layer "F.Cu") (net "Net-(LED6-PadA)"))
 (segment (start 37.277 35.7747) (end 42.4577 35.7747) (width 0.2) (layer "F.Cu") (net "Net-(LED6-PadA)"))
 (segment (start 35.8517 37.2) (end 37.277 35.7747) (width 0.2) (layer "F.Cu") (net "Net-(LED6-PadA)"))
 (segment (start 46.6983 34.65) (end 46.4905 34.65) (width 0.2) (layer "F.Cu") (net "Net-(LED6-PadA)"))
 (segment (start 47.6 34.65) (end 46.6983 34.65) (width 0.2) (layer "F.Cu") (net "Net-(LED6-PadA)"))
 (via (at 46.4905 34.65) (size 0.6) (drill 0.3) (layers "F.Cu" "B.Cu") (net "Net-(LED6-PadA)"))
 (via (at 42.4577 35.7747) (size 0.6) (drill 0.3) (layers "F.Cu" "B.Cu") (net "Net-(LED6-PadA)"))
 (segment (start 44.9237 36.2168) (end 46.4905 34.65) (width 0.2) (layer "B.Cu") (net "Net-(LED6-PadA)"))
 (segment (start 42.8998 36.2168) (end 44.9237 36.2168) (width 0.2) (layer "B.Cu") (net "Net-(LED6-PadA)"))
 (segment (start 42.4577 35.7747) (end 42.8998 36.2168) (width 0.2) (layer "B.Cu") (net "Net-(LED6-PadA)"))
 (segment (start 38.3837 29.9967) (end 37.982 30.3984) (width 0.2) (layer "F.Cu") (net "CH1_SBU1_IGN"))
 (segment (start 35.25 33.6) (end 35.25 32.9983) (width 0.2) (layer "F.Cu") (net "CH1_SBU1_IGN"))
 (segment (start 40.75 30) (end 40.1483 30) (width 0.2) (layer "F.Cu") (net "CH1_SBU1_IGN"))
 (segment (start 37.05 31.3001) (end 37.05 32.2018) (width 0.2) (layer "F.Cu") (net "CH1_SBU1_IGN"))
 (segment (start 28.73 31.27) (end 29.9715 30.0285) (width 0.2) (layer "F.Cu") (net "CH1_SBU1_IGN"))
 (segment (start 40.1483 30) (end 40.145 29.9967) (width 0.2) (layer "F.Cu") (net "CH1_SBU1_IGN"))
 (segment (start 36.0465 32.2018) (end 35.25 32.9983) (width 0.2) (layer "F.Cu") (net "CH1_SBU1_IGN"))
 (segment (start 29.9715 30.0285) (end 36.6801 30.0285) (width 0.2) (layer "F.Cu") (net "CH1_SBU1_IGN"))
 (segment (start 37.982 30.3984) (end 37.05 30.3984) (width 0.2) (layer "F.Cu") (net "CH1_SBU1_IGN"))
 (segment (start 37.05 32.2018) (end 36.0465 32.2018) (width 0.2) (layer "F.Cu") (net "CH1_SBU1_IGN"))
 (segment (start 40.145 29.9967) (end 38.3837 29.9967) (width 0.2) (layer "F.Cu") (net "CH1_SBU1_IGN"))
 (segment (start 36.6801 30.0285) (end 37.05 30.3984) (width 0.2) (layer "F.Cu") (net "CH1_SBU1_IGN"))
 (segment (start 37.05 31.3001) (end 37.05 30.3984) (width 0.2) (layer "F.Cu") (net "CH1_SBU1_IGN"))
 (segment (start 43.95 37.2) (end 43.3483 37.2) (width 0.2) (layer "F.Cu") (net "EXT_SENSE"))
 (segment (start 43.1266 36.9783) (end 43.012 36.9783) (width 0.2) (layer "F.Cu") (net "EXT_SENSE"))
 (segment (start 43.3483 37.2) (end 43.1266 36.9783) (width 0.2) (layer "F.Cu") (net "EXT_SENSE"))
 (via (at 43.012 36.9783) (size 0.6) (drill 0.3) (layers "F.Cu" "B.Cu") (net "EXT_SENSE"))
 (segment (start 42.5847 36.9783) (end 43.012 36.9783) (width 0.2) (layer "B.Cu") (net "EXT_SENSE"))
 (segment (start 31.27 28.73) (end 32.517 27.483) (width 0.2) (layer "B.Cu") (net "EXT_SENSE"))
 (segment (start 32.517 27.483) (end 36.3666 27.483) (width 0.2) (layer "B.Cu") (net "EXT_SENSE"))
 (segment (start 39.2585 30.3749) (end 39.2585 33.6521) (width 0.2) (layer "B.Cu") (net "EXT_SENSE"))
 (segment (start 39.2585 33.6521) (end 42.5847 36.9783) (width 0.2) (layer "B.Cu") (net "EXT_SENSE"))
 (segment (start 36.3666 27.483) (end 39.2585 30.3749) (width 0.2) (layer "B.Cu") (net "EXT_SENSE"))
 (segment (start 34.35 33.6) (end 34.35 34.2017) (width 0.2) (layer "F.Cu") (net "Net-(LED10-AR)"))
 (segment (start 43.45 34.6) (end 42.7483 34.6) (width 0.2) (layer "F.Cu") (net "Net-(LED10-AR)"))
 (segment (start 42.5977 34.7506) (end 42.7483 34.6) (width 0.2) (layer "F.Cu") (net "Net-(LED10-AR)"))
 (segment (start 34.35 34.2017) (end 34.8989 34.7506) (width 0.2) (layer "F.Cu") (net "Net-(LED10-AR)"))
 (segment (start 34.8989 34.7506) (end 42.5977 34.7506) (width 0.2) (layer "F.Cu") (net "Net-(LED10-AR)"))
 (segment (start 47.15 30) (end 47.15 30.6017) (width 0.2) (layer "F.Cu") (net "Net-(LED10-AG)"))
 (segment (start 44.6483 34.6784) (end 43.7571 35.5696) (width 0.2) (layer "F.Cu") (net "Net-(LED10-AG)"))
 (segment (start 45.35 34.6) (end 44.6483 34.6) (width 0.2) (layer "F.Cu") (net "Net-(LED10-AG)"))
 (segment (start 46.4878 30.6734) (end 46.5595 30.6017) (width 0.2) (layer "F.Cu") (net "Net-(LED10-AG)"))
 (segment (start 46.5595 30.6017) (end 47.15 30.6017) (width 0.2) (layer "F.Cu") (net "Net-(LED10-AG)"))
 (segment (start 44.6483 34.6) (end 44.6483 34.6784) (width 0.2) (layer "F.Cu") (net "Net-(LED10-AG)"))
 (via (at 46.4878 30.6734) (size 0.6) (drill 0.3) (layers "F.Cu" "B.Cu") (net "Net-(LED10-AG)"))
 (via (at 43.7571 35.5696) (size 0.6) (drill 0.3) (layers "F.Cu" "B.Cu") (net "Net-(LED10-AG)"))
 (segment (start 46.4878 32.8389) (end 43.7571 35.5696) (width 0.2) (layer "B.Cu") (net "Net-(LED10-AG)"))
 (segment (start 46.4878 30.6734) (end 46.4878 32.8389) (width 0.2) (layer "B.Cu") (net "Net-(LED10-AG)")))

